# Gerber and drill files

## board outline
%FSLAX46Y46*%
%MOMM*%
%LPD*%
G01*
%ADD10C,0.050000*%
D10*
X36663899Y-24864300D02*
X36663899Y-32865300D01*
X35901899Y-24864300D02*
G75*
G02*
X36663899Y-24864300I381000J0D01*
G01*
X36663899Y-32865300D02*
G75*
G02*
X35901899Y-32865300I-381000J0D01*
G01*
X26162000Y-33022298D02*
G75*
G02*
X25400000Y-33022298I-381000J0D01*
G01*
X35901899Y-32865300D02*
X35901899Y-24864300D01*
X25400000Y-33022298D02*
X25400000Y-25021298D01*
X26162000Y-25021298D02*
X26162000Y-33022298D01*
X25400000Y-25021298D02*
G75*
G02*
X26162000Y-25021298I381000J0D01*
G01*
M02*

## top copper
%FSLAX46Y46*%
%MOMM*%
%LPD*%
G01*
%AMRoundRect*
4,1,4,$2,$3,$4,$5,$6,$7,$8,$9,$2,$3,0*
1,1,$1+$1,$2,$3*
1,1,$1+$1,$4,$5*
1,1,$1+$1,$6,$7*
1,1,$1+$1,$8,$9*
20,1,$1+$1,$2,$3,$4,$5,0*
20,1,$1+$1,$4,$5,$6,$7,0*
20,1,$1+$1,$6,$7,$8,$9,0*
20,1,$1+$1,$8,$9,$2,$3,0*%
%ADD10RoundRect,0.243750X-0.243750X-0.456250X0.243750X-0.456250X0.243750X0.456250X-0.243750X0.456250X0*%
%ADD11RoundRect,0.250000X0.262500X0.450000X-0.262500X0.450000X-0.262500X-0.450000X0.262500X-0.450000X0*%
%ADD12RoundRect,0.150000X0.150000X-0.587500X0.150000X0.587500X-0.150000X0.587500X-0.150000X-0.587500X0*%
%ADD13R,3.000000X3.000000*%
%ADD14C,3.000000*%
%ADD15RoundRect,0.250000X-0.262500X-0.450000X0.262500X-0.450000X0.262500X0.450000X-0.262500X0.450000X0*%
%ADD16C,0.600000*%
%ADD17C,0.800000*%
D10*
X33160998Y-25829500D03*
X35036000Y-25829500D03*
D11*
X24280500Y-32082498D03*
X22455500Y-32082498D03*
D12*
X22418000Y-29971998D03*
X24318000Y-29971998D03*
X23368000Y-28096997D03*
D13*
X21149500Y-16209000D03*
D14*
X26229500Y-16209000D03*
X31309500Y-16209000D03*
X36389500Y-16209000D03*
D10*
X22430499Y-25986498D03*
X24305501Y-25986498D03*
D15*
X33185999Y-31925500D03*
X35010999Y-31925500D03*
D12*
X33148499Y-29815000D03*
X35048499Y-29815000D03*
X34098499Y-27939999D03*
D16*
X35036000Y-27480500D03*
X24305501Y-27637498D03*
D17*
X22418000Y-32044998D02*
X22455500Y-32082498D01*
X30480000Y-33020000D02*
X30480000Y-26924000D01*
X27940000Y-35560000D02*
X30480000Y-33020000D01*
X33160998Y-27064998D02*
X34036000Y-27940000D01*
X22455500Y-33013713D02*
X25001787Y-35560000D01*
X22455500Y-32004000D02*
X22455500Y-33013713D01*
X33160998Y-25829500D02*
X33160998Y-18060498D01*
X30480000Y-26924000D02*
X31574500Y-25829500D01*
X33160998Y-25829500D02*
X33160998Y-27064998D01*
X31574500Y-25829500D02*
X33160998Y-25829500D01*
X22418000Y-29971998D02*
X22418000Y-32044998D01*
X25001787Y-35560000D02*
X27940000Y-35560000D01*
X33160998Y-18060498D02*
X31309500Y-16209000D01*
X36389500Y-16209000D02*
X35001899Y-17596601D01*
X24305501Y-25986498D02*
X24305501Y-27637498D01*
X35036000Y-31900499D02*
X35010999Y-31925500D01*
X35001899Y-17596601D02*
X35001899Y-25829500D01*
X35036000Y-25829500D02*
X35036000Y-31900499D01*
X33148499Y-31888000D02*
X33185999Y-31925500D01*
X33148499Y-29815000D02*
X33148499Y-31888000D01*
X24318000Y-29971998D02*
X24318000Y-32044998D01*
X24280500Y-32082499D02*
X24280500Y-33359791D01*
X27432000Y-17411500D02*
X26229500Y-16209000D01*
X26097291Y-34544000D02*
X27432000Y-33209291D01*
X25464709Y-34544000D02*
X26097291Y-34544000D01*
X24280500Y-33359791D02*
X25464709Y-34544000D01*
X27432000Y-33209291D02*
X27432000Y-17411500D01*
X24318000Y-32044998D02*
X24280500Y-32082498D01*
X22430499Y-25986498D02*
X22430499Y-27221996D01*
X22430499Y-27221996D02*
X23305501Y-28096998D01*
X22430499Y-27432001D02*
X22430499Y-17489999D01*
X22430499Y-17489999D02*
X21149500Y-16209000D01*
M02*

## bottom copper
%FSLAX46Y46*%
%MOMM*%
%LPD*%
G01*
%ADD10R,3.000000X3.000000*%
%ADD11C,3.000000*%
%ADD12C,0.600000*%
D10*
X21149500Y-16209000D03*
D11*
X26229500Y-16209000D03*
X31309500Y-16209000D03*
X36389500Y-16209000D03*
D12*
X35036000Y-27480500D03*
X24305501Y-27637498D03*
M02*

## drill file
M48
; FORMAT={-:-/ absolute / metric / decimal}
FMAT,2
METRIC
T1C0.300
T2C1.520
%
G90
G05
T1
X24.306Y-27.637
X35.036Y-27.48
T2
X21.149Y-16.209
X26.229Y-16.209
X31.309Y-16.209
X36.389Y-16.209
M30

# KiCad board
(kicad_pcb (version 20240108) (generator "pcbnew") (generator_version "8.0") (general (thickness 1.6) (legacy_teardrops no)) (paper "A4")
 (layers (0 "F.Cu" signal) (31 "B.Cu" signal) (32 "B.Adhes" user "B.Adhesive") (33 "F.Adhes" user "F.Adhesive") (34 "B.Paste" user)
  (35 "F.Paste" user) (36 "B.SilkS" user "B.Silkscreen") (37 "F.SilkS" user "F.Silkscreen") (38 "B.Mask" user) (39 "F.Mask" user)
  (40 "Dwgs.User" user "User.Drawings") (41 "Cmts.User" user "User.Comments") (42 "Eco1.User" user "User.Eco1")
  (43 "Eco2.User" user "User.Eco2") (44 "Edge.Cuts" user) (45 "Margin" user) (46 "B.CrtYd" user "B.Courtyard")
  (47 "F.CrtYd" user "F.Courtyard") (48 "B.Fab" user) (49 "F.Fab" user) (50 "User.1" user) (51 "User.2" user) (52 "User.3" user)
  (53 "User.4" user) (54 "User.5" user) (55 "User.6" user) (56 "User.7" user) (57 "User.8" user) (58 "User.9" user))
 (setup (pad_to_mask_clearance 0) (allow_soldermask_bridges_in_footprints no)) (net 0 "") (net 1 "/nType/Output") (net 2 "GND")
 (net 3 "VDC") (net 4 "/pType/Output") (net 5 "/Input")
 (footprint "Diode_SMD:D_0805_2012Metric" (layer "F.Cu") (at 34.098499 25.8295)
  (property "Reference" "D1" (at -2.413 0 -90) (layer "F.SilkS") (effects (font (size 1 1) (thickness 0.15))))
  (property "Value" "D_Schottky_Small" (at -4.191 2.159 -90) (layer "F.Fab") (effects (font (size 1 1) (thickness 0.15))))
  (pad "1" smd roundrect (at -0.937501 0) (size 0.975 1.4) (layers "F.Cu" "F.Paste" "F.Mask") (roundrect_rratio 0.25)
   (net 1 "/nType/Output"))
  (pad "2" smd roundrect (at 0.937501 0) (size 0.975 1.4) (layers "F.Cu" "F.Paste" "F.Mask") (roundrect_rratio 0.25) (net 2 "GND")))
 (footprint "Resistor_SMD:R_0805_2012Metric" (layer "F.Cu") (at 23.368 32.082498 180)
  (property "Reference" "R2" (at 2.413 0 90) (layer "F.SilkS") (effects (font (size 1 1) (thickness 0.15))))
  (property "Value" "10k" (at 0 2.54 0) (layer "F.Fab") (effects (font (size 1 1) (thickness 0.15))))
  (pad "1" smd roundrect (at -0.9125 0 180) (size 1.025 1.4) (layers "F.Cu" "F.Paste" "F.Mask") (roundrect_rratio 0.243902) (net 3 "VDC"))
  (pad "2" smd roundrect (at 0.9125 0 180) (size 1.025 1.4) (layers "F.Cu" "F.Paste" "F.Mask") (roundrect_rratio 0.243902)
   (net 1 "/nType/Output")))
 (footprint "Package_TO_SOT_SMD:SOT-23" (layer "F.Cu") (at 23.368 29.034498 90)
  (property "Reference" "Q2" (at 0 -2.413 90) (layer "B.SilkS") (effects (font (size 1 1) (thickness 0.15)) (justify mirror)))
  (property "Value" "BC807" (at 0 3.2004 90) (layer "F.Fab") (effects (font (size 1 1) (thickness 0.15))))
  (pad "1" smd roundrect (at -0.9375 -0.95 90) (size 1.475 0.6) (layers "F.Cu" "F.Paste" "F.Mask") (roundrect_rratio 0.25)
   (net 1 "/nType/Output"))
  (pad "2" smd roundrect (at -0.9375 0.95 90) (size 1.475 0.6) (layers "F.Cu" "F.Paste" "F.Mask") (roundrect_rratio 0.25) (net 3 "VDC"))
  (pad "3" smd roundrect (at 0.937501 0 90) (size 1.475 0.6) (layers "F.Cu" "F.Paste" "F.Mask") (roundrect_rratio 0.25)
   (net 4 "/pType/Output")))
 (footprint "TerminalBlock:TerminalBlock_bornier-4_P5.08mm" (layer "F.Cu") (at 21.1495 16.209)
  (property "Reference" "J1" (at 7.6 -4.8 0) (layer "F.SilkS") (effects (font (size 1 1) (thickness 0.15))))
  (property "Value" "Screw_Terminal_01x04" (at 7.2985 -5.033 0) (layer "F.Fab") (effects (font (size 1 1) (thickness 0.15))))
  (pad "1" thru_hole rect (at 0 0) (size 3 3) (drill 1.52) (layers "*.Cu" "*.Mask") (remove_unused_layers no) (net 4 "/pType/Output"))
  (pad "2" thru_hole circle (at 5.08 0) (size 3 3) (drill 1.52) (layers "*.Cu" "*.Mask") (remove_unused_layers no) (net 3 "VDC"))
  (pad "3" thru_hole circle (at 10.16 0) (size 3 3) (drill 1.52) (layers "*.Cu" "*.Mask") (remove_unused_layers no) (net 1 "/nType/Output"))
  (pad "4" thru_hole circle (at 15.24 0) (size 3 3) (drill 1.52) (layers "*.Cu" "*.Mask") (remove_unused_layers no) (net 2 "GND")))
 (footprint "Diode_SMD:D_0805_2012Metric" (layer "F.Cu") (at 23.368 25.986498)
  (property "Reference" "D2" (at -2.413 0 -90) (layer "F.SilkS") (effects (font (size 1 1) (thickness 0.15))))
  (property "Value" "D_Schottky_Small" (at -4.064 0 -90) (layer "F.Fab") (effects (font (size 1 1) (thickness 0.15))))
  (pad "1" smd roundrect (at -0.937501 0) (size 0.975 1.4) (layers "F.Cu" "F.Paste" "F.Mask") (roundrect_rratio 0.25)
   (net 4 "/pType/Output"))
  (pad "2" smd roundrect (at 0.937501 0) (size 0.975 1.4) (layers "F.Cu" "F.Paste" "F.Mask") (roundrect_rratio 0.25) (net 2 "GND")))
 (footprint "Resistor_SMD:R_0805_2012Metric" (layer "F.Cu") (at 34.098499 31.9255)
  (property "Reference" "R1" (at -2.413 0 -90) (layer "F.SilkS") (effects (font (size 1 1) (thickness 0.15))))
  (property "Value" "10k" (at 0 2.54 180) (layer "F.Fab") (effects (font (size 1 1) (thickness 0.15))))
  (pad "1" smd roundrect (at -0.9125 0) (size 1.025 1.4) (layers "F.Cu" "F.Paste" "F.Mask") (roundrect_rratio 0.243902) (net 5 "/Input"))
  (pad "2" smd roundrect (at 0.9125 0) (size 1.025 1.4) (layers "F.Cu" "F.Paste" "F.Mask") (roundrect_rratio 0.243902) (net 2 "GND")))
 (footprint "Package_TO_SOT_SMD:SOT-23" (layer "F.Cu") (at 34.098499 28.8775 90)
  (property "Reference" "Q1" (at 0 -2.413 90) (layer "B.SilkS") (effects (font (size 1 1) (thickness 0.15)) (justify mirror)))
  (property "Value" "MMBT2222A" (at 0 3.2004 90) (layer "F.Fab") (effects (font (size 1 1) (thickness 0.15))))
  (pad "1" smd roundrect (at -0.9375 -0.95 90) (size 1.475 0.6) (layers "F.Cu" "F.Paste" "F.Mask") (roundrect_rratio 0.25) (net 5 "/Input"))
  (pad "2" smd roundrect (at -0.9375 0.95 90) (size 1.475 0.6) (layers "F.Cu" "F.Paste" "F.Mask") (roundrect_rratio 0.25) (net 2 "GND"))
  (pad "3" smd roundrect (at 0.937501 0 90) (size 1.475 0.6) (layers "F.Cu" "F.Paste" "F.Mask") (roundrect_rratio 0.25)
   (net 1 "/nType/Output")))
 (gr_line (start 36.663899 24.8643) (end 36.663899 32.8653) (stroke (width 0.05) (type default)) (layer "Edge.Cuts"))
 (gr_arc (start 35.901899 24.8643) (mid 36.282899 24.4833) (end 36.663899 24.8643) (stroke (width 0.05) (type default)) (layer "Edge.Cuts"))
 (gr_arc (start 36.663899 32.8653) (mid 36.282899 33.2463) (end 35.901899 32.8653) (stroke (width 0.05) (type default)) (layer "Edge.Cuts"))
 (gr_arc (start 26.162 33.022298) (mid 25.781 33.403298) (end 25.4 33.022298) (stroke (width 0.05) (type default)) (layer "Edge.Cuts"))
 (gr_line (start 35.901899 32.8653) (end 35.901899 24.8643) (stroke (width 0.05) (type default)) (layer "Edge.Cuts"))
 (gr_line (start 25.4 33.022298) (end 25.4 25.021298) (stroke (width 0.05) (type default)) (layer "Edge.Cuts"))
 (gr_line (start 26.162 25.021298) (end 26.162 33.022298) (stroke (width 0.05) (type default)) (layer "Edge.Cuts"))
 (gr_arc (start 25.4 25.021298) (mid 25.781 24.640298) (end 26.162 25.021298) (stroke (width 0.05) (type default)) (layer "Edge.Cuts"))
 (segment (start 22.418 32.044998) (end 22.4555 32.082498) (width 0.8) (layer "F.Cu") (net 1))
 (segment (start 30.48 33.02) (end 30.48 26.924) (width 0.8) (layer "F.Cu") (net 1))
 (segment (start 27.94 35.56) (end 30.48 33.02) (width 0.8) (layer "F.Cu") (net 1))
 (segment (start 33.160998 27.064998) (end 34.036 27.94) (width 0.8) (layer "F.Cu") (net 1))
 (segment (start 22.4555 33.013713) (end 25.001787 35.56) (width 0.8) (layer "F.Cu") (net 1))
 (segment (start 22.4555 32.004) (end 22.4555 33.013713) (width 0.8) (layer "F.Cu") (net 1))
 (segment (start 33.160998 25.8295) (end 33.160998 18.060498) (width 0.8) (layer "F.Cu") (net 1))
 (segment (start 30.48 26.924) (end 31.5745 25.8295) (width 0.8) (layer "F.Cu") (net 1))
 (segment (start 33.160998 25.8295) (end 33.160998 27.064998) (width 0.8) (layer "F.Cu") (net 1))
 (segment (start 31.5745 25.8295) (end 33.160998 25.8295) (width 0.8) (layer "F.Cu") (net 1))
 (segment (start 22.418 29.971998) (end 22.418 32.044998) (width 0.8) (layer "F.Cu") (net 1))
 (segment (start 25.001787 35.56) (end 27.94 35.56) (width 0.8) (layer "F.Cu") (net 1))
 (segment (start 33.160998 18.060498) (end 31.3095 16.209) (width 0.8) (layer "F.Cu") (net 1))
 (segment (start 36.3895 16.209) (end 35.001899 17.596601) (width 0.8) (layer "F.Cu") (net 2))
 (segment (start 24.305501 25.986498) (end 24.305501 27.637498) (width 0.8) (layer "F.Cu") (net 2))
 (segment (start 35.036 31.900499) (end 35.010999 31.9255) (width 0.8) (layer "F.Cu") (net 2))
 (segment (start 35.001899 17.596601) (end 35.001899 25.8295) (width 0.8) (layer "F.Cu") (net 2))
 (segment (start 35.036 25.8295) (end 35.036 31.900499) (width 0.8) (layer "F.Cu") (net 2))
 (via (at 35.036 27.4805) (size 0.6) (drill 0.3) (layers "F.Cu" "B.Cu") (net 2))
 (via (at 24.305501 27.637498) (size 0.6) (drill 0.3) (layers "F.Cu" "B.Cu") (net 2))
 (segment (start 33.148499 31.888) (end 33.185999 31.9255) (width 0.8) (layer "F.Cu") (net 5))
 (segment (start 33.148499 29.815) (end 33.148499 31.888) (width 0.8) (layer "F.Cu") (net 5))
 (segment (start 24.318 29.971998) (end 24.318 32.044998) (width 0.8) (layer "F.Cu") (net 3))
 (segment (start 24.2805 32.082499) (end 24.2805 33.359791) (width 0.8) (layer "F.Cu") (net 3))
 (segment (start 27.432 17.4115) (end 26.2295 16.209) (width 0.8) (layer "F.Cu") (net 3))
 (segment (start 26.097291 34.544) (end 27.432 33.209291) (width 0.8) (layer "F.Cu") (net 3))
 (segment (start 25.464709 34.544) (end 26.097291 34.544) (width 0.8) (layer "F.Cu") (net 3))
 (segment (start 24.2805 33.359791) (end 25.464709 34.544) (width 0.8) (layer "F.Cu") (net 3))
 (segment (start 27.432 33.209291) (end 27.432 17.4115) (width 0.8) (layer "F.Cu") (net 3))
 (segment (start 24.318 32.044998) (end 24.2805 32.082498) (width 0.8) (layer "F.Cu") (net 3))
 (segment (start 22.430499 25.986498) (end 22.430499 27.221996) (width 0.8) (layer "F.Cu") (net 4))
 (segment (start 22.430499 27.221996) (end 23.305501 28.096998) (width 0.8) (layer "F.Cu") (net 4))
 (segment (start 22.430499 27.432001) (end 22.430499 17.489999) (width 0.8) (layer "F.Cu") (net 4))
 (segment (start 22.430499 17.489999) (end 21.1495 16.209) (width 0.8) (layer "F.Cu") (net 4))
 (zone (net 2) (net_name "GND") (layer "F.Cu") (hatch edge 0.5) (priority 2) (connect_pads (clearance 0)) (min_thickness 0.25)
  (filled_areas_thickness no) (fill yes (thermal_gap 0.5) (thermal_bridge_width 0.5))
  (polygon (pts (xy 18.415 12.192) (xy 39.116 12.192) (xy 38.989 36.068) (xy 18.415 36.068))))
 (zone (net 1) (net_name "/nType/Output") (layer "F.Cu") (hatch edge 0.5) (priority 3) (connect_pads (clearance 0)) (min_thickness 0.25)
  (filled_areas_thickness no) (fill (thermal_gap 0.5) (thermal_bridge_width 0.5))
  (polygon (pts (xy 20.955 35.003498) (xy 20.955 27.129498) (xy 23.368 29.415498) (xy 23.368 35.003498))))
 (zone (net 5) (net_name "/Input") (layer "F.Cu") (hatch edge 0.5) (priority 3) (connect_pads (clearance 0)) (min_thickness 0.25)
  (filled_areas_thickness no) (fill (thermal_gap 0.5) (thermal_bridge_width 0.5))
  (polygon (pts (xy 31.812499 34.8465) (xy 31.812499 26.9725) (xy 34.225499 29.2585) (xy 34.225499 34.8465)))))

